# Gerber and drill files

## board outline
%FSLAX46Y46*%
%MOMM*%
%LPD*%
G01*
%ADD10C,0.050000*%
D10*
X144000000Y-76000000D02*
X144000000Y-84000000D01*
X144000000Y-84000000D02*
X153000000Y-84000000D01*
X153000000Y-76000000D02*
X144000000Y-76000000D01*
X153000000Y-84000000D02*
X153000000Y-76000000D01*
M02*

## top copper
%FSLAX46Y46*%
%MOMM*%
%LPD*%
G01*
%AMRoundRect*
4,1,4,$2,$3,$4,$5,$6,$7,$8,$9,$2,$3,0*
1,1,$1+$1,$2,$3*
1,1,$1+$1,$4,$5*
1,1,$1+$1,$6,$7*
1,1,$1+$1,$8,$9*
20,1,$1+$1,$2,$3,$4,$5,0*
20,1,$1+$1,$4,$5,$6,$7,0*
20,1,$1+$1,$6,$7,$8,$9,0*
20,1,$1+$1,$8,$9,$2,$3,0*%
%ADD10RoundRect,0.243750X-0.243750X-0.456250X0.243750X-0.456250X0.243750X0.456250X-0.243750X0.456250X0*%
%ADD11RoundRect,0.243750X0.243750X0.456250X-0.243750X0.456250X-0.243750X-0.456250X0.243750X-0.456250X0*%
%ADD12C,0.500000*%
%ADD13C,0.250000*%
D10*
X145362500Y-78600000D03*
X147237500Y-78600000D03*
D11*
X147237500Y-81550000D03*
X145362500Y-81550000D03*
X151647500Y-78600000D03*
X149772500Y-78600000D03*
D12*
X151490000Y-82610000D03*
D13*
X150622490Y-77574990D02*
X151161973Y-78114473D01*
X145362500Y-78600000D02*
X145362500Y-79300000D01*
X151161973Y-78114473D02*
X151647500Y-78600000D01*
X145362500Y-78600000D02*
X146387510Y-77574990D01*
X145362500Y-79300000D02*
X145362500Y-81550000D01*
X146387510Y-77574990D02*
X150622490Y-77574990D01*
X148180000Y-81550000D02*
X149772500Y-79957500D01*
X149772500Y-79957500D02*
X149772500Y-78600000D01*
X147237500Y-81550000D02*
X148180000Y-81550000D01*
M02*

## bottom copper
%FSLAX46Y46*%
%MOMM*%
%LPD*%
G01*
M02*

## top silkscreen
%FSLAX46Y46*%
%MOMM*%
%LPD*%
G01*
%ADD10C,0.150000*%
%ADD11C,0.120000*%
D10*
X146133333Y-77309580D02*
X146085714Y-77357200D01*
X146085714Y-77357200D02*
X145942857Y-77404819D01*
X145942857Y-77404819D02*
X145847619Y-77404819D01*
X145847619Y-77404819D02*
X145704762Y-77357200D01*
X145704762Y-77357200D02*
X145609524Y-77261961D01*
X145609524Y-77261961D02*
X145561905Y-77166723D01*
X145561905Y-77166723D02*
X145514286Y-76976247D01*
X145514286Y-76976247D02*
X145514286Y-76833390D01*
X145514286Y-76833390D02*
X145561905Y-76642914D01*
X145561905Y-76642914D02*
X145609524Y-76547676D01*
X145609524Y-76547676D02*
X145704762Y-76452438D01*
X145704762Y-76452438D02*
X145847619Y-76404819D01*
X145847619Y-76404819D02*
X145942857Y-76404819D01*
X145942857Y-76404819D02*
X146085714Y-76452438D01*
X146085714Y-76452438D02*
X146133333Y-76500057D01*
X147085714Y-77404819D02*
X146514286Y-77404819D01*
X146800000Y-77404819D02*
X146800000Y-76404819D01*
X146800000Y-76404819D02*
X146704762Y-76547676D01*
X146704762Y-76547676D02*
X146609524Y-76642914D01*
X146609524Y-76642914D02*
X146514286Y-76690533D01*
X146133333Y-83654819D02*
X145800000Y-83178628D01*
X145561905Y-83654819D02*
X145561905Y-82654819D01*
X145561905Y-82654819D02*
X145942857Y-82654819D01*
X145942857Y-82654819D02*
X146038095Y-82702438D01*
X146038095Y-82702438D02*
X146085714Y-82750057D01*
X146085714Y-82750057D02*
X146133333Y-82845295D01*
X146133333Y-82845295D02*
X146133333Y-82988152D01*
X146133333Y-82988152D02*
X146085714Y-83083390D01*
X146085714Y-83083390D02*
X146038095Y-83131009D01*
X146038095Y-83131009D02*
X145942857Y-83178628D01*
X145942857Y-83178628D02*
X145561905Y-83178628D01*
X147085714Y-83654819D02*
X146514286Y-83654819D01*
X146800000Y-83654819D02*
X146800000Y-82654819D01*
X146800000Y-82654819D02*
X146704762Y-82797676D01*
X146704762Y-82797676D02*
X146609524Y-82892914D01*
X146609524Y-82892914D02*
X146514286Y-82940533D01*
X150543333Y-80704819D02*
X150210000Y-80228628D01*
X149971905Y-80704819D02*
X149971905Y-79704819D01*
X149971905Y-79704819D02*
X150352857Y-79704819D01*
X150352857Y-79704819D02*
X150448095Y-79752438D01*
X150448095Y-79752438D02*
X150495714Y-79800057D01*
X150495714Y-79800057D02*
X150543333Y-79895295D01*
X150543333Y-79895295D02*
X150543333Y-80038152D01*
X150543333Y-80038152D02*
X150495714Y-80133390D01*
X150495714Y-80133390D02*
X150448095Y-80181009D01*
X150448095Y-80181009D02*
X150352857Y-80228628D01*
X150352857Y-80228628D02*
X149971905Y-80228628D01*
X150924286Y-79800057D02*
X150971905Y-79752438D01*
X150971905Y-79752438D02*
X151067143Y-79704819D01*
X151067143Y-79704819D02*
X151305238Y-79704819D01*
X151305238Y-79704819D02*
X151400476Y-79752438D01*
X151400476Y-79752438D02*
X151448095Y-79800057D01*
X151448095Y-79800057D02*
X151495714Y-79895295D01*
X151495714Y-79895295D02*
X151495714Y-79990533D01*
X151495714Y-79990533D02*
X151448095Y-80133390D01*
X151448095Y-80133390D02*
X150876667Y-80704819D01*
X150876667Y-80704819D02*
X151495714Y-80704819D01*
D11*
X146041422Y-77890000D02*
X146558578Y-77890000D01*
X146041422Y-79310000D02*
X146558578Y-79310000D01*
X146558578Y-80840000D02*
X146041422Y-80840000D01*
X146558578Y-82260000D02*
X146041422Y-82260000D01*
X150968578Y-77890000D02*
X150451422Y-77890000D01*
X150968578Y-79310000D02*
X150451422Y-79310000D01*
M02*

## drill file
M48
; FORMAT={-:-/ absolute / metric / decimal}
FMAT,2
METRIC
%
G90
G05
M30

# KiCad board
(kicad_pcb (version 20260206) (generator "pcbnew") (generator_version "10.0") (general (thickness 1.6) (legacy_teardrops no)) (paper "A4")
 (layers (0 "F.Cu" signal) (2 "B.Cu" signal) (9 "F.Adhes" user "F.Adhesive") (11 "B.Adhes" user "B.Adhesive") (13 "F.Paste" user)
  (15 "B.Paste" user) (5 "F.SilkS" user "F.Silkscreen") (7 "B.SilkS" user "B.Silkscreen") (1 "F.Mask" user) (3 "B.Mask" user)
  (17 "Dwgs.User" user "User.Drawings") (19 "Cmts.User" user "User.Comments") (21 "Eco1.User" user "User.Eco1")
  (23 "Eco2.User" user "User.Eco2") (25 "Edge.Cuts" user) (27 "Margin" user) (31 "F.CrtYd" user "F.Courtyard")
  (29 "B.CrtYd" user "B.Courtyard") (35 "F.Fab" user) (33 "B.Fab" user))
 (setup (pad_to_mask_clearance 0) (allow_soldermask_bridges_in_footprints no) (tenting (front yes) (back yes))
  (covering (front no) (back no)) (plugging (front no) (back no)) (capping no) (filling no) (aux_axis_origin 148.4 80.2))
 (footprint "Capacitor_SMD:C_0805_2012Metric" (layer "F.Cu") (at 146.3 78.6)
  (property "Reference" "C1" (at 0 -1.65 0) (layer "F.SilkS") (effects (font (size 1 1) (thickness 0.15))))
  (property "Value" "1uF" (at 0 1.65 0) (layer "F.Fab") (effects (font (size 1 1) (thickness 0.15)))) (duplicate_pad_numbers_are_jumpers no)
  (fp_line (start -0.258578 -0.71) (end 0.258578 -0.71) (stroke (width 0.12) (type solid)) (layer "F.SilkS"))
  (fp_line (start -0.258578 0.71) (end 0.258578 0.71) (stroke (width 0.12) (type solid)) (layer "F.SilkS"))
  (pad "1" smd roundrect (at -0.9375 0) (size 0.975 1.4) (layers "F.Cu" "F.Mask" "F.Paste") (roundrect_rratio 0.25) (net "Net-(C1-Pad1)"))
  (pad "2" smd roundrect (at 0.9375 0) (size 0.975 1.4) (layers "F.Cu" "F.Mask" "F.Paste") (roundrect_rratio 0.25) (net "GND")))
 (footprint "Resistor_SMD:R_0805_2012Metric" (layer "F.Cu") (at 146.3 81.55 180)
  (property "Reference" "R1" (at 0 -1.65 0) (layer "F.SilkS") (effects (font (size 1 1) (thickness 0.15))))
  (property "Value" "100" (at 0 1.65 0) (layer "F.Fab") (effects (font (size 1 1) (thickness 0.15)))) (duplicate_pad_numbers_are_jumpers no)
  (fp_line (start -0.258578 0.71) (end 0.258578 0.71) (stroke (width 0.12) (type solid)) (layer "F.SilkS"))
  (fp_line (start -0.258578 -0.71) (end 0.258578 -0.71) (stroke (width 0.12) (type solid)) (layer "F.SilkS"))
  (pad "1" smd roundrect (at -0.9375 0 180) (size 0.975 1.4) (layers "F.Cu" "F.Mask" "F.Paste") (roundrect_rratio 0.25) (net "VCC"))
  (pad "2" smd roundrect (at 0.9375 0 180) (size 0.975 1.4) (layers "F.Cu" "F.Mask" "F.Paste") (roundrect_rratio 0.25) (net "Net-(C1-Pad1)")))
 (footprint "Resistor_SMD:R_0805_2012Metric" (layer "F.Cu") (at 150.71 78.6 180)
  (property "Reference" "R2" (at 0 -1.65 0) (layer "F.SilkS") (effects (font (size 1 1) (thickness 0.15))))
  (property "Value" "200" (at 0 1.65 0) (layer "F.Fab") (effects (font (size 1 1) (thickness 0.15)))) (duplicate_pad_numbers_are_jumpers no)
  (fp_line (start -0.258578 0.71) (end 0.258578 0.71) (stroke (width 0.12) (type solid)) (layer "F.SilkS"))
  (fp_line (start -0.258578 -0.71) (end 0.258578 -0.71) (stroke (width 0.12) (type solid)) (layer "F.SilkS"))
  (pad "1" smd roundrect (at -0.9375 0 180) (size 0.975 1.4) (layers "F.Cu" "F.Mask" "F.Paste") (roundrect_rratio 0.25)
   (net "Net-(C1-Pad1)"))
  (pad "2" smd roundrect (at 0.9375 0 180) (size 0.975 1.4) (layers "F.Cu" "F.Mask" "F.Paste") (roundrect_rratio 0.25) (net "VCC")))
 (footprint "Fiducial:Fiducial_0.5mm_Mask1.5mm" (layer "F.Cu") (at 151.49 82.61)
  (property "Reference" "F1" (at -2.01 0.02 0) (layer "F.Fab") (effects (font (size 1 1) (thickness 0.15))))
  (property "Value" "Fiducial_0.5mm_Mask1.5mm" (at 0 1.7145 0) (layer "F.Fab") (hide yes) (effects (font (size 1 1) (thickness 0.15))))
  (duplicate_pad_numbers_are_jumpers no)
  (pad "" smd circle (at 0 0) (size 0.5 0.5) (layers "F.Cu" "F.Mask") (solder_mask_margin 0.5) (clearance 0.5)))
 (gr_line (start 144 76) (end 144 84) (stroke (width 0.05) (type solid)) (layer "Edge.Cuts"))
 (gr_line (start 144 84) (end 153 84) (stroke (width 0.05) (type solid)) (layer "Edge.Cuts"))
 (gr_line (start 153 76) (end 144 76) (stroke (width 0.05) (type solid)) (layer "Edge.Cuts"))
 (gr_line (start 153 84) (end 153 76) (stroke (width 0.05) (type solid)) (layer "Edge.Cuts"))
 (segment (start 150.62249 77.57499) (end 151.161973 78.114473) (width 0.25) (layer "F.Cu") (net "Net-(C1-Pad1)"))
 (segment (start 145.3625 78.6) (end 145.3625 79.3) (width 0.25) (layer "F.Cu") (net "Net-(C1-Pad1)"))
 (segment (start 151.161973 78.114473) (end 151.6475 78.6) (width 0.25) (layer "F.Cu") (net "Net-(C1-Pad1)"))
 (segment (start 145.3625 78.6) (end 146.38751 77.57499) (width 0.25) (layer "F.Cu") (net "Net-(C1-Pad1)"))
 (segment (start 145.3625 79.3) (end 145.3625 81.55) (width 0.25) (layer "F.Cu") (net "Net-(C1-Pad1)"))
 (segment (start 146.38751 77.57499) (end 150.62249 77.57499) (width 0.25) (layer "F.Cu") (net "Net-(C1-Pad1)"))
 (segment (start 148.18 81.55) (end 149.7725 79.9575) (width 0.25) (layer "F.Cu") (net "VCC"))
 (segment (start 149.7725 79.9575) (end 149.7725 78.6) (width 0.25) (layer "F.Cu") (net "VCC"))
 (segment (start 147.2375 81.55) (end 148.18 81.55) (width 0.25) (layer "F.Cu") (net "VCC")))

